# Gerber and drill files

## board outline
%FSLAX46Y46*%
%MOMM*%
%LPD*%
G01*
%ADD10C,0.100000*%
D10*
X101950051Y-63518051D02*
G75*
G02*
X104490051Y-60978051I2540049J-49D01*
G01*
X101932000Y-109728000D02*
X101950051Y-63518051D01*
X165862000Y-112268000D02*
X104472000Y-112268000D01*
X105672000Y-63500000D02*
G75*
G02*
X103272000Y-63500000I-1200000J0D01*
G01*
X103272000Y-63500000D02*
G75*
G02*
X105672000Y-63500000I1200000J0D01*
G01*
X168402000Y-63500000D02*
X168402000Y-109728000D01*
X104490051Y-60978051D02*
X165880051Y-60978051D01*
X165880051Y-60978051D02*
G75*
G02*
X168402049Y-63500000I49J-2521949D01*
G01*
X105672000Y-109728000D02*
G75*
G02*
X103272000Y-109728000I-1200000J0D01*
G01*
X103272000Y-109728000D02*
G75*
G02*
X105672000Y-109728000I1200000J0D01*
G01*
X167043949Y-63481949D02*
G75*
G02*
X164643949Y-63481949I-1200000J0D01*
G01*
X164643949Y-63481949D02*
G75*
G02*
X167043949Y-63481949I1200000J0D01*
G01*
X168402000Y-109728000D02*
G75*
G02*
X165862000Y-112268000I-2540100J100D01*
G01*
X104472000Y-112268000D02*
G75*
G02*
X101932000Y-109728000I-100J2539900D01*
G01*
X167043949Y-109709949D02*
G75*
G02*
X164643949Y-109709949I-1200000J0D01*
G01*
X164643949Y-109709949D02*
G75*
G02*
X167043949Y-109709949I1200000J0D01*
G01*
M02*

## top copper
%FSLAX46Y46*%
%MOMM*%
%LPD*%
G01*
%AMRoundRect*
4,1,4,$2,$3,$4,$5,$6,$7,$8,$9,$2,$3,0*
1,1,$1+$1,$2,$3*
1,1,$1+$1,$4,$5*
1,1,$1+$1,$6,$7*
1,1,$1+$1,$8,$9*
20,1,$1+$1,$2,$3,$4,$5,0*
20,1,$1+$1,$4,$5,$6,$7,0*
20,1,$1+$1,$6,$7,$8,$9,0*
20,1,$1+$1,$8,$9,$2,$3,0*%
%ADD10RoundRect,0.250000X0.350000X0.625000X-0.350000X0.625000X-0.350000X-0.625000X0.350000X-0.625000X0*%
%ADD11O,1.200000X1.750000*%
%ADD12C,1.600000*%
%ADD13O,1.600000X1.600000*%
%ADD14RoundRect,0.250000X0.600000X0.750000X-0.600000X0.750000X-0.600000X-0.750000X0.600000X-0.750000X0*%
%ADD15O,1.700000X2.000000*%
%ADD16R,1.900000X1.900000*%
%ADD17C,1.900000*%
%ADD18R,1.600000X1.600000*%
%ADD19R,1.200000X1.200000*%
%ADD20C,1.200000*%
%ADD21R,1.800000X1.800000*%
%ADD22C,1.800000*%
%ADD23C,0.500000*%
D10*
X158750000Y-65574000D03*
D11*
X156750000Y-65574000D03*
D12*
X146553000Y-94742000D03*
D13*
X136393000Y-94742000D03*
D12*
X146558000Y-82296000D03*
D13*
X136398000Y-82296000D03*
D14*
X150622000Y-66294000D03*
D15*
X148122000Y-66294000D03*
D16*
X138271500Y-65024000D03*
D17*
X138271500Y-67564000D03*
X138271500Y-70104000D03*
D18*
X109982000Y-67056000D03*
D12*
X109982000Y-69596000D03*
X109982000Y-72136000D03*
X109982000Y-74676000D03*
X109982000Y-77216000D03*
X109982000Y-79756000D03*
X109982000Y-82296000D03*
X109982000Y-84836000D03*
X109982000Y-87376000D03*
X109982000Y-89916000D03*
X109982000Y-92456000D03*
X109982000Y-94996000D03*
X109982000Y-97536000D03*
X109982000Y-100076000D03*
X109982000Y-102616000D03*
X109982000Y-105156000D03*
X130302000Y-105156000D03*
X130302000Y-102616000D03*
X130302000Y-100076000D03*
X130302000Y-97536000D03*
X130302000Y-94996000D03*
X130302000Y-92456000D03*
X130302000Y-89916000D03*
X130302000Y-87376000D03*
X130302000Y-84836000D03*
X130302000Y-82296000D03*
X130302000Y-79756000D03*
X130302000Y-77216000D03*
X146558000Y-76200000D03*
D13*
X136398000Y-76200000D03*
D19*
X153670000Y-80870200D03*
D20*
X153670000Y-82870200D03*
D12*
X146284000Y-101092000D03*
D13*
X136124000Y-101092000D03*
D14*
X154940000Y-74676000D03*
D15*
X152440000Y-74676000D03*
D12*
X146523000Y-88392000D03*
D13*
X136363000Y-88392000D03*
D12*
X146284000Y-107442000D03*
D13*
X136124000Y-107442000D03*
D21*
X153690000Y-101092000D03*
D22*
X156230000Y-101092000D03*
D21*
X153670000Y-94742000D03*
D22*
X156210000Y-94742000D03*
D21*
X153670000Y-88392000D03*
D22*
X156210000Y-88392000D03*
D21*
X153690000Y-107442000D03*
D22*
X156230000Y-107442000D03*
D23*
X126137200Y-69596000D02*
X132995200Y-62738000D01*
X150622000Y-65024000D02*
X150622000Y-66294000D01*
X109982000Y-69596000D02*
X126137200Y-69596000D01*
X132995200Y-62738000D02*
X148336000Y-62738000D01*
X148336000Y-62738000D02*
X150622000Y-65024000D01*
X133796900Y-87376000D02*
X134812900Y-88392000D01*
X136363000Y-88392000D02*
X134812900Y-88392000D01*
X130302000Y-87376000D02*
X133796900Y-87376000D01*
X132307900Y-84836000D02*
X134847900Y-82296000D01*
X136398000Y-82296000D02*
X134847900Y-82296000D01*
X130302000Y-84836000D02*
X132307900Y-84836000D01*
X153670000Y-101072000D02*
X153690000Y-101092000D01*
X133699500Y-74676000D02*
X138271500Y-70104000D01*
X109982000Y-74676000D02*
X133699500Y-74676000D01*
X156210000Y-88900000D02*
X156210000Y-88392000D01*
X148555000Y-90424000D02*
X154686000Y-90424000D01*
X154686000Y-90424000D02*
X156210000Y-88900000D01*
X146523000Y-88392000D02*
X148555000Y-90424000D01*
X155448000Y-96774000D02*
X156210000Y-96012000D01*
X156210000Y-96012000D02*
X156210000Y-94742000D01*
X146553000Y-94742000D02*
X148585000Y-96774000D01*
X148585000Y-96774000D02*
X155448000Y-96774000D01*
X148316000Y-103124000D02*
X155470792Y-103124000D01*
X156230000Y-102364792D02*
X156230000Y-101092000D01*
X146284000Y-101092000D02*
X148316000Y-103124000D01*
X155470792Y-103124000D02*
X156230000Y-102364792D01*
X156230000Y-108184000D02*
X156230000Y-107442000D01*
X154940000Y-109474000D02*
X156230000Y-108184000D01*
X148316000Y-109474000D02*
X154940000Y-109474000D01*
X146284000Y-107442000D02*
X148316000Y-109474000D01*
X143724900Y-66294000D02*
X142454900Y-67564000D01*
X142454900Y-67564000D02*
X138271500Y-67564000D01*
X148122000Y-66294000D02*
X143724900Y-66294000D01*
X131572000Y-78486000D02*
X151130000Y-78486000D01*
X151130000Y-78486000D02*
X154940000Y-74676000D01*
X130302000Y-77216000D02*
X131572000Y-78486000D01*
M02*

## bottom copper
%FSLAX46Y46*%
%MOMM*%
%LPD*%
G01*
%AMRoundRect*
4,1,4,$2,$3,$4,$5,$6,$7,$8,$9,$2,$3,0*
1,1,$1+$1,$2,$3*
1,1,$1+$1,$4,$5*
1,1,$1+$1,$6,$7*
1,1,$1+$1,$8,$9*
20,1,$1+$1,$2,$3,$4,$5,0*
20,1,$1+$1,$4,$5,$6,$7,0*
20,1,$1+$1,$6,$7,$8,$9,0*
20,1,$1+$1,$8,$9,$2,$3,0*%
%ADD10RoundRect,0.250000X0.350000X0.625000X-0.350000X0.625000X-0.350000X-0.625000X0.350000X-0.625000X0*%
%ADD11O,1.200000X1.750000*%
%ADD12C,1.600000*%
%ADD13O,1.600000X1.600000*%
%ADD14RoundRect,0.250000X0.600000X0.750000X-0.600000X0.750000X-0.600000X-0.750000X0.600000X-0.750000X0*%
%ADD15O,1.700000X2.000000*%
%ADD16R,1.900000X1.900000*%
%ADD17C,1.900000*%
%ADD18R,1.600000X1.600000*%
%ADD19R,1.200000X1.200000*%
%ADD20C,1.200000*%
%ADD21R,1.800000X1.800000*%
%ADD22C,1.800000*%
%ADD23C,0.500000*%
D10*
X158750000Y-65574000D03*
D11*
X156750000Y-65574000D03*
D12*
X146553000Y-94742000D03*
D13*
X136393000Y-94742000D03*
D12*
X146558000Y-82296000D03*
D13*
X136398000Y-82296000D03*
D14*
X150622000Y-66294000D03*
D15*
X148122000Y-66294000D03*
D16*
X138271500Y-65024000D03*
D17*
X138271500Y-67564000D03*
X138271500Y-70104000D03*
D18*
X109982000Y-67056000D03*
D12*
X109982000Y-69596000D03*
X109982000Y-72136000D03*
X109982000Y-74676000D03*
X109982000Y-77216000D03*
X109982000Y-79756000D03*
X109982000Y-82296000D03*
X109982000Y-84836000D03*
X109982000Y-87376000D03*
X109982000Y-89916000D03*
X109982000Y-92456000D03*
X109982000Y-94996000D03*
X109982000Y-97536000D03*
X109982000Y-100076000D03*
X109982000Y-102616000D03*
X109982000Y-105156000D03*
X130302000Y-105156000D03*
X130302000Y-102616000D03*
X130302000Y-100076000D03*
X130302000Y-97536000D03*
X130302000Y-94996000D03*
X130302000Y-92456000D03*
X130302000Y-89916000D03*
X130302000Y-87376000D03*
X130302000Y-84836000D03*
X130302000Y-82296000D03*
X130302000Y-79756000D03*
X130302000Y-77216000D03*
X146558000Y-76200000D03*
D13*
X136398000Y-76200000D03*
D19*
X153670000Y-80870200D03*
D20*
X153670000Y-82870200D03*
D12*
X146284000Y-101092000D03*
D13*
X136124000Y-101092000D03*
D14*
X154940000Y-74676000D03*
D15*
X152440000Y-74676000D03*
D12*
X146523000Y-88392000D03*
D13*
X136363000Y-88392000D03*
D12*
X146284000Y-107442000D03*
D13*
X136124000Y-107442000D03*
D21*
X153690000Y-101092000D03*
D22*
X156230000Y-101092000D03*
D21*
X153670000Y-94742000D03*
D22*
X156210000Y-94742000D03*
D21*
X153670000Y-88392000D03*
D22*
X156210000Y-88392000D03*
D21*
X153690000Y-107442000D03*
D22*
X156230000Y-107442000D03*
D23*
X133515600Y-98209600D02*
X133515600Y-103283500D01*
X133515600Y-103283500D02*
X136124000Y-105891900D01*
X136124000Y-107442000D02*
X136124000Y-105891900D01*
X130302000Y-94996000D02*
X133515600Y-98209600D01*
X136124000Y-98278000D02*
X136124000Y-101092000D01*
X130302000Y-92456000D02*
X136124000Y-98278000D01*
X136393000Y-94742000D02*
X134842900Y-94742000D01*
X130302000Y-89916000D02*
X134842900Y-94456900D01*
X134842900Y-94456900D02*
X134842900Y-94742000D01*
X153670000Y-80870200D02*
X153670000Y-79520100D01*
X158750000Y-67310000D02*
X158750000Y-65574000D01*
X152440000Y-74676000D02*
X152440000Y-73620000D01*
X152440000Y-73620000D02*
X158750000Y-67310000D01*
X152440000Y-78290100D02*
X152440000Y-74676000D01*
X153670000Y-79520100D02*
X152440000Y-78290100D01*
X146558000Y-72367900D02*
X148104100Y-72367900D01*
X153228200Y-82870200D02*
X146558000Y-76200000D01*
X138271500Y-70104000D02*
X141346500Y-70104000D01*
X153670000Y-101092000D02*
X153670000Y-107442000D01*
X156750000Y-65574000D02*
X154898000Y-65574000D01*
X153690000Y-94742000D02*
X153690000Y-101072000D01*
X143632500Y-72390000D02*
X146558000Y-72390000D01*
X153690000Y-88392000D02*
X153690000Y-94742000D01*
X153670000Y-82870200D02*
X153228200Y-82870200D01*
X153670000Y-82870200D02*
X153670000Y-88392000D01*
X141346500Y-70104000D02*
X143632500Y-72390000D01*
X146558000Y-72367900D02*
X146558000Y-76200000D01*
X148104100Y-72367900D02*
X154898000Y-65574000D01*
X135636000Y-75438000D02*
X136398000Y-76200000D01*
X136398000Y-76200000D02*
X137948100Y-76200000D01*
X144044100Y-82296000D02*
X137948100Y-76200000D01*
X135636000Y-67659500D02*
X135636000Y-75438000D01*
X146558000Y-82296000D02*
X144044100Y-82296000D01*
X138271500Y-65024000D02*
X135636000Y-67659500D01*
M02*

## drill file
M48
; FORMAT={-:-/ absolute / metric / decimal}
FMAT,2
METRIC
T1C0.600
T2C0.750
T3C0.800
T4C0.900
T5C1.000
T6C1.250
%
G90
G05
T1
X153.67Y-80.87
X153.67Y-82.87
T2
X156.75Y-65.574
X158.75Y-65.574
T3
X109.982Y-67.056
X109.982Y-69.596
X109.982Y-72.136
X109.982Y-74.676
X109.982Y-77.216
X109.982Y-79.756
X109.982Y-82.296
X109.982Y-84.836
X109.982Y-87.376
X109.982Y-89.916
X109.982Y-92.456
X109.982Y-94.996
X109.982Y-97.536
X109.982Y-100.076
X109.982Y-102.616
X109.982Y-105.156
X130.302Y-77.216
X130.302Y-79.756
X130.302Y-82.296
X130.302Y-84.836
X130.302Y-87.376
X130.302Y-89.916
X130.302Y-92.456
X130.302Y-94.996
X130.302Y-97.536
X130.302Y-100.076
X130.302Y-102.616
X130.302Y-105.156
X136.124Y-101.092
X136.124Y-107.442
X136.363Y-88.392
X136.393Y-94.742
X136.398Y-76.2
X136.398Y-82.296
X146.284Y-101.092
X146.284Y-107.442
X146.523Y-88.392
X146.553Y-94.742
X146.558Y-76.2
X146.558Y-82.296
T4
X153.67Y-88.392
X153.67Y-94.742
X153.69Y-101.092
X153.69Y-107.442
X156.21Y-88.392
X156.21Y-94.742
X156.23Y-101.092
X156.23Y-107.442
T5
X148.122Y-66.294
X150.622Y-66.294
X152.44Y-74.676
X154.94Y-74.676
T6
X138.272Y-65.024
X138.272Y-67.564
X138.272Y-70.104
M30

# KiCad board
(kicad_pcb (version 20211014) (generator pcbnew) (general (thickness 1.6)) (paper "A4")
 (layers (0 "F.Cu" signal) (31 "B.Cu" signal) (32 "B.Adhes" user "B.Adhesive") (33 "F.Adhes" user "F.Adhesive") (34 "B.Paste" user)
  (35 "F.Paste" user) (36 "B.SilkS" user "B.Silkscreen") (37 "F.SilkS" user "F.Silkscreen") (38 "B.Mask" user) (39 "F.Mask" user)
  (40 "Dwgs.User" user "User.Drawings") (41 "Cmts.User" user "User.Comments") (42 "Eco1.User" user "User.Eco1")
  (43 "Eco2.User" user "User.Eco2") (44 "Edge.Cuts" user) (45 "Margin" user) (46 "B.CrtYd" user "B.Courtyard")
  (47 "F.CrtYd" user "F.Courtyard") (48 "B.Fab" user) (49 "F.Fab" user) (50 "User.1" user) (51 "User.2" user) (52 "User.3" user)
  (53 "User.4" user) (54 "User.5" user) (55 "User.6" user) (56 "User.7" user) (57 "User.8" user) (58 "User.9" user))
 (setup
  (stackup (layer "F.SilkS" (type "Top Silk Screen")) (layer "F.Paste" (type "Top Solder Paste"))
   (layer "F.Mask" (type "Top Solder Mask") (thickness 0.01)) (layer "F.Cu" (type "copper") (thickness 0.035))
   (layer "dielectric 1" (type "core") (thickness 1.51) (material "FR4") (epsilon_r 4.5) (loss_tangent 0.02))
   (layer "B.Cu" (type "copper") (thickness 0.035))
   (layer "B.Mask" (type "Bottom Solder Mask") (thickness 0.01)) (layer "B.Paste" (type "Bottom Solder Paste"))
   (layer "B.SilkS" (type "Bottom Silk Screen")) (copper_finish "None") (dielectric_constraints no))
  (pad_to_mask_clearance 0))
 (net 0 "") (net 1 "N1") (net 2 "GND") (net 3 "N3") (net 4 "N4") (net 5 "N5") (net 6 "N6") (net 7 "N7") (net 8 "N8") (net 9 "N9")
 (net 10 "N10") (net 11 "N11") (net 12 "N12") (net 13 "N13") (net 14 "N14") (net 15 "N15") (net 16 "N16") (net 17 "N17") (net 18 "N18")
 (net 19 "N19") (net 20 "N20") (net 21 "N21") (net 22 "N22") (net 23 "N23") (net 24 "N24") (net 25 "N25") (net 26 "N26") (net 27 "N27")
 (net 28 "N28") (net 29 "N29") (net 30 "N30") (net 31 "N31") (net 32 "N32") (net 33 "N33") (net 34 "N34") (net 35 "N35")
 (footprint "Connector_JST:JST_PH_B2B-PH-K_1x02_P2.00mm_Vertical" (layer "F.Cu") (at 158.75 65.574 180)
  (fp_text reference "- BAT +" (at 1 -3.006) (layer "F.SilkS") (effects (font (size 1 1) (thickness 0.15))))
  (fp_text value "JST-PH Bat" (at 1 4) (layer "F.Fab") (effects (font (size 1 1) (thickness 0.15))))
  (pad "1" thru_hole roundrect (at 0 0 180) (size 1.2 1.75) (drill 0.75) (layers *.Cu *.Mask) (roundrect_rratio 0.208333) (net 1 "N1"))
  (pad "2" thru_hole oval (at 2 0 180) (size 1.2 1.75) (drill 0.75) (layers *.Cu *.Mask) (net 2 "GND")))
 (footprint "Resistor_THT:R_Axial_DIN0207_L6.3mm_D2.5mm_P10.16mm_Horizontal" (layer "F.Cu") (at 146.553 94.742 180)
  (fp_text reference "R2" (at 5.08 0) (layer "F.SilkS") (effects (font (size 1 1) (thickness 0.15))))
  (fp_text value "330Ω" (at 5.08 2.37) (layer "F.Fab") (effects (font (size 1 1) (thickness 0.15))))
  (pad "1" thru_hole circle (at 0 0 180) (size 1.6 1.6) (drill 0.8) (layers *.Cu *.Mask) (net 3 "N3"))
  (pad "2" thru_hole oval (at 10.16 0 180) (size 1.6 1.6) (drill 0.8) (layers *.Cu *.Mask) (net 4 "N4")))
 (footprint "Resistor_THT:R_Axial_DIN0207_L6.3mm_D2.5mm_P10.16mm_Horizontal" (layer "F.Cu") (at 146.558 82.296 180)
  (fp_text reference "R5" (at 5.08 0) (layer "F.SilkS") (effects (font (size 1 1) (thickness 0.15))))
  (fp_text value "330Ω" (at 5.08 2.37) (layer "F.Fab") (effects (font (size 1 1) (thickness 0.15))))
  (pad "1" thru_hole circle (at 0 0 180) (size 1.6 1.6) (drill 0.8) (layers *.Cu *.Mask) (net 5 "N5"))
  (pad "2" thru_hole oval (at 10.16 0 180) (size 1.6 1.6) (drill 0.8) (layers *.Cu *.Mask) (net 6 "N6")))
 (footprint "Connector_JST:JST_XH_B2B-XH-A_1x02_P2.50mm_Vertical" (layer "F.Cu") (at 150.622 66.294 180)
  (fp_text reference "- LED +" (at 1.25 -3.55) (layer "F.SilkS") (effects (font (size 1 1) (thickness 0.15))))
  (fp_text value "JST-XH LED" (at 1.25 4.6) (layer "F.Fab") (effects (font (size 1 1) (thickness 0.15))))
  (pad "1" thru_hole roundrect (at 0 0 180) (size 1.7 2) (drill 1) (layers *.Cu *.Mask) (roundrect_rratio 0.147059) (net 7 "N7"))
  (pad "2" thru_hole oval (at 2.5 0 180) (size 1.7 2) (drill 1) (layers *.Cu *.Mask) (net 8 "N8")))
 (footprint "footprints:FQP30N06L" (layer "F.Cu") (at 138.684 67.564)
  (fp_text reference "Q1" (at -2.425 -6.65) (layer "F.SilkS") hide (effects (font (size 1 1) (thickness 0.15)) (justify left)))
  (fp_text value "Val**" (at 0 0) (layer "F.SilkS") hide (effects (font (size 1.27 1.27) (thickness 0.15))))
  (pad "1" thru_hole rect (at -0.4125 -2.54) (size 1.9 1.9) (drill 1.25) (layers *.Cu *.Mask) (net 5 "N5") (thermal_width 0.45))
  (pad "2" thru_hole circle (at -0.4125 0) (size 1.9 1.9) (drill 1.25) (layers *.Cu *.Mask) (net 8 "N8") (thermal_width 0.45))
  (pad "3" thru_hole circle (at -0.4125 2.54) (size 1.9 1.9) (drill 1.25) (layers *.Cu *.Mask) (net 2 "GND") (thermal_width 0.45)))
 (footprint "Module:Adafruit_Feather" (layer "F.Cu") (at 109.982 67.056)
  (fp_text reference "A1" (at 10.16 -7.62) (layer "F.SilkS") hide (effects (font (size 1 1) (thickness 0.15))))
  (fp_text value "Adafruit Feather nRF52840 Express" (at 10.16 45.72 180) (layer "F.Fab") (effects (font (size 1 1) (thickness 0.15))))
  (pad "1" thru_hole rect (at 0 0 180) (size 1.6 1.6) (drill 0.8) (layers *.Cu *.Mask) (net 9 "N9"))
  (pad "2" thru_hole circle (at 0 2.54 180) (size 1.6 1.6) (drill 0.8) (layers *.Cu *.Mask) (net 7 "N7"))
  (pad "3" thru_hole circle (at 0 5.08 180) (size 1.6 1.6) (drill 0.8) (layers *.Cu *.Mask) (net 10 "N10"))
  (pad "4" thru_hole circle (at 0 7.62 180) (size 1.6 1.6) (drill 0.8) (layers *.Cu *.Mask) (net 2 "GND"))
  (pad "5" thru_hole circle (at 0 10.16 180) (size 1.6 1.6) (drill 0.8) (layers *.Cu *.Mask) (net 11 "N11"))
  (pad "6" thru_hole circle (at 0 12.7 180) (size 1.6 1.6) (drill 0.8) (layers *.Cu *.Mask) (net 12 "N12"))
  (pad "7" thru_hole circle (at 0 15.24 180) (size 1.6 1.6) (drill 0.8) (layers *.Cu *.Mask) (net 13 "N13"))
  (pad "8" thru_hole circle (at 0 17.78 180) (size 1.6 1.6) (drill 0.8) (layers *.Cu *.Mask) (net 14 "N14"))
  (pad "9" thru_hole circle (at 0 20.32 180) (size 1.6 1.6) (drill 0.8) (layers *.Cu *.Mask) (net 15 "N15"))
  (pad "10" thru_hole circle (at 0 22.86 180) (size 1.6 1.6) (drill 0.8) (layers *.Cu *.Mask) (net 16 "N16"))
  (pad "11" thru_hole circle (at 0 25.4 180) (size 1.6 1.6) (drill 0.8) (layers *.Cu *.Mask) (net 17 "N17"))
  (pad "12" thru_hole circle (at 0 27.94 180) (size 1.6 1.6) (drill 0.8) (layers *.Cu *.Mask) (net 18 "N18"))
  (pad "13" thru_hole circle (at 0 30.48 180) (size 1.6 1.6) (drill 0.8) (layers *.Cu *.Mask) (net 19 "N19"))
  (pad "14" thru_hole circle (at 0 33.02 180) (size 1.6 1.6) (drill 0.8) (layers *.Cu *.Mask) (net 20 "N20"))
  (pad "15" thru_hole circle (at 0 35.56 180) (size 1.6 1.6) (drill 0.8) (layers *.Cu *.Mask) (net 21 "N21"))
  (pad "16" thru_hole circle (at 0 38.1 180) (size 1.6 1.6) (drill 0.8) (layers *.Cu *.Mask) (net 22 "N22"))
  (pad "17" thru_hole circle (at 20.32 38.1 180) (size 1.6 1.6) (drill 0.8) (layers *.Cu *.Mask) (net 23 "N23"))
  (pad "18" thru_hole circle (at 20.32 35.56 180) (size 1.6 1.6) (drill 0.8) (layers *.Cu *.Mask) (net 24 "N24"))
  (pad "19" thru_hole circle (at 20.32 33.02 180) (size 1.6 1.6) (drill 0.8) (layers *.Cu *.Mask) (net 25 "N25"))
  (pad "20" thru_hole circle (at 20.32 30.48 180) (size 1.6 1.6) (drill 0.8) (layers *.Cu *.Mask) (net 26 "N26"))
  (pad "21" thru_hole circle (at 20.32 27.94 180) (size 1.6 1.6) (drill 0.8) (layers *.Cu *.Mask) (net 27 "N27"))
  (pad "22" thru_hole circle (at 20.32 25.4 180) (size 1.6 1.6) (drill 0.8) (layers *.Cu *.Mask) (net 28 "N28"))
  (pad "23" thru_hole circle (at 20.32 22.86 180) (size 1.6 1.6) (drill 0.8) (layers *.Cu *.Mask) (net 4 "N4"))
  (pad "24" thru_hole circle (at 20.32 20.32 180) (size 1.6 1.6) (drill 0.8) (layers *.Cu *.Mask) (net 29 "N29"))
  (pad "25" thru_hole circle (at 20.32 17.78 180) (size 1.6 1.6) (drill 0.8) (layers *.Cu *.Mask) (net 6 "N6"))
  (pad "26" thru_hole circle (at 20.32 15.24 180) (size 1.6 1.6) (drill 0.8) (layers *.Cu *.Mask) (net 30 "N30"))
  (pad "27" thru_hole circle (at 20.32 12.7 180) (size 1.6 1.6) (drill 0.8) (layers *.Cu *.Mask) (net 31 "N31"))
  (pad "28" thru_hole circle (at 20.32 10.16 180) (size 1.6 1.6) (drill 0.8) (layers *.Cu *.Mask) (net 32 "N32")))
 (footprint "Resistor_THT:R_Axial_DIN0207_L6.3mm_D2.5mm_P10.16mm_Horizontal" (layer "F.Cu") (at 146.558 76.2 180)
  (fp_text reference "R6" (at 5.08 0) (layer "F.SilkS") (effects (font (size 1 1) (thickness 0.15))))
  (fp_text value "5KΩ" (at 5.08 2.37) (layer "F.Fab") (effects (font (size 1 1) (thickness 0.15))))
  (pad "1" thru_hole circle (at 0 0 180) (size 1.6 1.6) (drill 0.8) (layers *.Cu *.Mask) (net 2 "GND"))
  (pad "2" thru_hole oval (at 10.16 0 180) (size 1.6 1.6) (drill 0.8) (layers *.Cu *.Mask) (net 5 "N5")))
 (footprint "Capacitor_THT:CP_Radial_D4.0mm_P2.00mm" (layer "F.Cu") (at 153.67 80.8702 -90)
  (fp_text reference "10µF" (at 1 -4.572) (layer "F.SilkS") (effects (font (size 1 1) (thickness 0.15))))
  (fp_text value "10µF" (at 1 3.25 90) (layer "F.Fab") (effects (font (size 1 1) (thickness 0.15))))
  (pad "1" thru_hole rect (at 0 0 270) (size 1.2 1.2) (drill 0.6) (layers *.Cu *.Mask) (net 1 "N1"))
  (pad "2" thru_hole circle (at 2 0 270) (size 1.2 1.2) (drill 0.6) (layers *.Cu *.Mask) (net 2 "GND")))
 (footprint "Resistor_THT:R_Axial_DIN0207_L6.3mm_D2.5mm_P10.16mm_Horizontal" (layer "F.Cu") (at 146.284 101.092 180)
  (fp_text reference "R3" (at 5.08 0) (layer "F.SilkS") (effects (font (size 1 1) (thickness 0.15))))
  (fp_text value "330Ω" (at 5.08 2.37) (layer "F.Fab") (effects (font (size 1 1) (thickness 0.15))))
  (pad "1" thru_hole circle (at 0 0 180) (size 1.6 1.6) (drill 0.8) (layers *.Cu *.Mask) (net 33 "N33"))
  (pad "2" thru_hole oval (at 10.16 0 180) (size 1.6 1.6) (drill 0.8) (layers *.Cu *.Mask) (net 28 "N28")))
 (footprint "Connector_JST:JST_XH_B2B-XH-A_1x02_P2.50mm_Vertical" (layer "F.Cu") (at 154.94 74.676 180)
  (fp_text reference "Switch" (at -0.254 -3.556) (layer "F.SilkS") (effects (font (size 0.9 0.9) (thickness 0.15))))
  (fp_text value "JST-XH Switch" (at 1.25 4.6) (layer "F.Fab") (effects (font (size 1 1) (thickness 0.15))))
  (pad "1" thru_hole roundrect (at 0 0 180) (size 1.7 2) (drill 1) (layers *.Cu *.Mask) (roundrect_rratio 0.147059) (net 32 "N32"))
  (pad "2" thru_hole oval (at 2.5 0 180) (size 1.7 2) (drill 1) (layers *.Cu *.Mask) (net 1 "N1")))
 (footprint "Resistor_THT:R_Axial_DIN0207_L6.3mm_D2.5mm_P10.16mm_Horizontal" (layer "F.Cu") (at 146.523 88.392 180)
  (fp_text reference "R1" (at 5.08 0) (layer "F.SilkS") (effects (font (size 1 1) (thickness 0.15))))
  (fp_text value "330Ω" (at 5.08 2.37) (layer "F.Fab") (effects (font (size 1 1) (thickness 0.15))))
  (pad "1" thru_hole circle (at 0 0 180) (size 1.6 1.6) (drill 0.8) (layers *.Cu *.Mask) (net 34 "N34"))
  (pad "2" thru_hole oval (at 10.16 0 180) (size 1.6 1.6) (drill 0.8) (layers *.Cu *.Mask) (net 29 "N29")))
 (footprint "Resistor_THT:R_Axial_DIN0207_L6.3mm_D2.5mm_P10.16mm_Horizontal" (layer "F.Cu") (at 146.284 107.442 180)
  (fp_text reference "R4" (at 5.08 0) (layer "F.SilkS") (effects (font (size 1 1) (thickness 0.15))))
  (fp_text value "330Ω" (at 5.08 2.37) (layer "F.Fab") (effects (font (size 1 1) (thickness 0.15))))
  (pad "1" thru_hole circle (at 0 0 180) (size 1.6 1.6) (drill 0.8) (layers *.Cu *.Mask) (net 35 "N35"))
  (pad "2" thru_hole oval (at 10.16 0 180) (size 1.6 1.6) (drill 0.8) (layers *.Cu *.Mask) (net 27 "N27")))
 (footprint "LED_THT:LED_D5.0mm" (layer "B.Cu") (at 153.69 101.092)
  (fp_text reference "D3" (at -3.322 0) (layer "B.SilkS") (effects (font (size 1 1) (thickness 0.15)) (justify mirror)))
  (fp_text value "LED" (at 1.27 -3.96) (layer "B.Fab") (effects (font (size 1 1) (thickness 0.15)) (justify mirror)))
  (pad "1" thru_hole rect (at 0 0) (size 1.8 1.8) (drill 0.9) (layers *.Cu *.Mask) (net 2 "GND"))
  (pad "2" thru_hole circle (at 2.54 0) (size 1.8 1.8) (drill 0.9) (layers *.Cu *.Mask) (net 33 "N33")))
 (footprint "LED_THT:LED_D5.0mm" (layer "B.Cu") (at 153.67 94.742)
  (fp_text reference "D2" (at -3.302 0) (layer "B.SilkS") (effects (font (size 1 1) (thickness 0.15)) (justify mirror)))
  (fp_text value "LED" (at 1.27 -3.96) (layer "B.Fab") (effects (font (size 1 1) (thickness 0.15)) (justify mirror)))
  (pad "1" thru_hole rect (at 0 0) (size 1.8 1.8) (drill 0.9) (layers *.Cu *.Mask) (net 2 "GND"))
  (pad "2" thru_hole circle (at 2.54 0) (size 1.8 1.8) (drill 0.9) (layers *.Cu *.Mask) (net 3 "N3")))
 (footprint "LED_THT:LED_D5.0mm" (layer "B.Cu") (at 153.67 88.392)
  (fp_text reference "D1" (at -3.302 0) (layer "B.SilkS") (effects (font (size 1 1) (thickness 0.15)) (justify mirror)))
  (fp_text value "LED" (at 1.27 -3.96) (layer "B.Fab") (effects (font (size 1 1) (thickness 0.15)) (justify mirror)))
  (pad "1" thru_hole rect (at 0 0) (size 1.8 1.8) (drill 0.9) (layers *.Cu *.Mask) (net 2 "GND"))
  (pad "2" thru_hole circle (at 2.54 0) (size 1.8 1.8) (drill 0.9) (layers *.Cu *.Mask) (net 34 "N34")))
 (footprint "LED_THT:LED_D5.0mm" (layer "B.Cu") (at 153.69 107.442)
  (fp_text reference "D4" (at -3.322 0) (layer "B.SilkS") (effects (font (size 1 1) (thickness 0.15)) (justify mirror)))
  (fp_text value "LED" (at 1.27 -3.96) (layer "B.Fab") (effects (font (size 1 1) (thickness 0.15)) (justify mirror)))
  (pad "1" thru_hole rect (at 0 0) (size 1.8 1.8) (drill 0.9) (layers *.Cu *.Mask) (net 2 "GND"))
  (pad "2" thru_hole circle (at 2.54 0) (size 1.8 1.8) (drill 0.9) (layers *.Cu *.Mask) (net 35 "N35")))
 (gr_arc (start 101.950051 63.518051) (mid 102.694 61.722) (end 104.490051 60.978051) (layer "Edge.Cuts") (width 0.1))
 (gr_line (start 101.932 109.728) (end 101.950051 63.518051) (layer "Edge.Cuts") (width 0.1))
 (gr_line (start 165.862 112.268) (end 104.472 112.268) (layer "Edge.Cuts") (width 0.1))
 (gr_circle (center 104.472 63.5) (end 105.672 63.5) (layer "Edge.Cuts") (width 0.1) (fill none))
 (gr_line (start 168.402 63.5) (end 168.402 109.728) (layer "Edge.Cuts") (width 0.1))
 (gr_line (start 104.490051 60.978051) (end 165.880051 60.978051) (layer "Edge.Cuts") (width 0.1))
 (gr_arc (start 165.880051 60.978051) (mid 167.663352 61.716699) (end 168.402 63.5) (layer "Edge.Cuts") (width 0.1))
 (gr_circle (center 104.472 109.728) (end 105.672 109.728) (layer "Edge.Cuts") (width 0.1) (fill none))
 (gr_circle (center 165.843949 63.481949) (end 167.043949 63.481949) (layer "Edge.Cuts") (width 0.1) (fill none))
 (gr_arc (start 168.402 109.728) (mid 167.658034 111.52402) (end 165.862 112.268) (layer "Edge.Cuts") (width 0.1))
 (gr_arc (start 104.472 112.268) (mid 102.6759 111.524072) (end 101.932 109.728) (layer "Edge.Cuts") (width 0.1))
 (gr_circle (center 165.843949 109.709949) (end 167.043949 109.709949) (layer "Edge.Cuts") (width 0.1) (fill none))
 (segment (start 126.1372 69.596) (end 132.9952 62.738) (width 0.5) (layer "F.Cu") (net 7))
 (segment (start 150.622 65.024) (end 150.622 66.294) (width 0.5) (layer "F.Cu") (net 7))
 (segment (start 109.982 69.596) (end 126.1372 69.596) (width 0.5) (layer "F.Cu") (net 7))
 (segment (start 132.9952 62.738) (end 148.336 62.738) (width 0.5) (layer "F.Cu") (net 7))
 (segment (start 148.336 62.738) (end 150.622 65.024) (width 0.5) (layer "F.Cu") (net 7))
 (segment (start 133.5156 98.2096) (end 133.5156 103.2835) (width 0.5) (layer "B.Cu") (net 27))
 (segment (start 133.5156 103.2835) (end 136.124 105.8919) (width 0.5) (layer "B.Cu") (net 27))
 (segment (start 136.124 107.442) (end 136.124 105.8919) (width 0.5) (layer "B.Cu") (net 27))
 (segment (start 130.302 94.996) (end 133.5156 98.2096) (width 0.5) (layer "B.Cu") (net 27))
 (segment (start 136.124 98.278) (end 136.124 101.092) (width 0.5) (layer "B.Cu") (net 28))
 (segment (start 130.302 92.456) (end 136.124 98.278) (width 0.5) (layer "B.Cu") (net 28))
 (segment (start 136.393 94.742) (end 134.8429 94.742) (width 0.5) (layer "B.Cu") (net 4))
 (segment (start 130.302 89.916) (end 134.8429 94.4569) (width 0.5) (layer "B.Cu") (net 4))
 (segment (start 134.8429 94.4569) (end 134.8429 94.742) (width 0.5) (layer "B.Cu") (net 4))
 (segment (start 133.7969 87.376) (end 134.8129 88.392) (width 0.5) (layer "F.Cu") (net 29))
 (segment (start 136.363 88.392) (end 134.8129 88.392) (width 0.5) (layer "F.Cu") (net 29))
 (segment (start 130.302 87.376) (end 133.7969 87.376) (width 0.5) (layer "F.Cu") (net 29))
 (segment (start 132.3079 84.836) (end 134.8479 82.296) (width 0.5) (layer "F.Cu") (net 6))
 (segment (start 136.398 82.296) (end 134.8479 82.296) (width 0.5) (layer "F.Cu") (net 6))
 (segment (start 130.302 84.836) (end 132.3079 84.836) (width 0.5) (layer "F.Cu") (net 6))
 (segment (start 153.67 80.8702) (end 153.67 79.5201) (width 0.5) (layer "B.Cu") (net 1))
 (segment (start 158.75 67.31) (end 158.75 65.574) (width 0.5) (layer "B.Cu") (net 1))
 (segment (start 152.44 74.676) (end 152.44 73.62) (width 0.5) (layer "B.Cu") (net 1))
 (segment (start 152.44 73.62) (end 158.75 67.31) (width 0.5) (layer "B.Cu") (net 1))
 (segment (start 152.44 78.2901) (end 152.44 74.676) (width 0.5) (layer "B.Cu") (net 1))
 (segment (start 153.67 79.5201) (end 152.44 78.2901) (width 0.5) (layer "B.Cu") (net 1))
 (segment (start 153.67 101.072) (end 153.69 101.092) (width 0.5) (layer "F.Cu") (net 2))
 (segment (start 133.6995 74.676) (end 138.2715 70.104) (width 0.5) (layer "F.Cu") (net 2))
 (segment (start 109.982 74.676) (end 133.6995 74.676) (width 0.5) (layer "F.Cu") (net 2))
 (segment (start 146.558 72.3679) (end 148.1041 72.3679) (width 0.5) (layer "B.Cu") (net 2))
 (segment (start 153.2282 82.8702) (end 146.558 76.2) (width 0.5) (layer "B.Cu") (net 2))
 (segment (start 138.2715 70.104) (end 141.3465 70.104) (width 0.5) (layer "B.Cu") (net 2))
 (segment (start 153.67 101.092) (end 153.67 107.442) (width 0.5) (layer "B.Cu") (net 2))
 (segment (start 156.75 65.574) (end 154.898 65.574) (width 0.5) (layer "B.Cu") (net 2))
 (segment (start 153.69 94.742) (end 153.69 101.072) (width 0.5) (layer "B.Cu") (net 2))
 (segment (start 143.6325 72.39) (end 146.558 72.39) (width 0.5) (layer "B.Cu") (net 2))
 (segment (start 153.69 88.392) (end 153.69 94.742) (width 0.5) (layer "B.Cu") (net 2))
 (segment (start 153.67 82.8702) (end 153.2282 82.8702) (width 0.5) (layer "B.Cu") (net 2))
 (segment (start 153.67 82.8702) (end 153.67 88.392) (width 0.5) (layer "B.Cu") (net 2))
 (segment (start 141.3465 70.104) (end 143.6325 72.39) (width 0.5) (layer "B.Cu") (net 2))
 (segment (start 146.558 72.3679) (end 146.558 76.2) (width 0.5) (layer "B.Cu") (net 2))
 (segment (start 148.1041 72.3679) (end 154.898 65.574) (width 0.5) (layer "B.Cu") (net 2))
 (segment (start 156.21 88.9) (end 156.21 88.392) (width 0.5) (layer "F.Cu") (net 34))
 (segment (start 148.555 90.424) (end 154.686 90.424) (width 0.5) (layer "F.Cu") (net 34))
 (segment (start 154.686 90.424) (end 156.21 88.9) (width 0.5) (layer "F.Cu") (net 34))
 (segment (start 146.523 88.392) (end 148.555 90.424) (width 0.5) (layer "F.Cu") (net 34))
 (segment (start 155.448 96.774) (end 156.21 96.012) (width 0.5) (layer "F.Cu") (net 3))
 (segment (start 156.21 96.012) (end 156.21 94.742) (width 0.5) (layer "F.Cu") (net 3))
 (segment (start 146.553 94.742) (end 148.585 96.774) (width 0.5) (layer "F.Cu") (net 3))
 (segment (start 148.585 96.774) (end 155.448 96.774) (width 0.5) (layer "F.Cu") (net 3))
 (segment (start 148.316 103.124) (end 155.470792 103.124) (width 0.5) (layer "F.Cu") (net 33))
 (segment (start 156.23 102.364792) (end 156.23 101.092) (width 0.5) (layer "F.Cu") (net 33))
 (segment (start 146.284 101.092) (end 148.316 103.124) (width 0.5) (layer "F.Cu") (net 33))
 (segment (start 155.470792 103.124) (end 156.23 102.364792) (width 0.5) (layer "F.Cu") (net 33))
 (segment (start 156.23 108.184) (end 156.23 107.442) (width 0.5) (layer "F.Cu") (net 35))
 (segment (start 154.94 109.474) (end 156.23 108.184) (width 0.5) (layer "F.Cu") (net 35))
 (segment (start 148.316 109.474) (end 154.94 109.474) (width 0.5) (layer "F.Cu") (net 35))
 (segment (start 146.284 107.442) (end 148.316 109.474) (width 0.5) (layer "F.Cu") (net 35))
 (segment (start 143.7249 66.294) (end 142.4549 67.564) (width 0.5) (layer "F.Cu") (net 8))
 (segment (start 142.4549 67.564) (end 138.2715 67.564) (width 0.5) (layer "F.Cu") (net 8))
 (segment (start 148.122 66.294) (end 143.7249 66.294) (width 0.5) (layer "F.Cu") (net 8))
 (segment (start 135.636 75.438) (end 136.398 76.2) (width 0.5) (layer "B.Cu") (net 5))
 (segment (start 136.398 76.2) (end 137.9481 76.2) (width 0.5) (layer "B.Cu") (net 5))
 (segment (start 144.0441 82.296) (end 137.9481 76.2) (width 0.5) (layer "B.Cu") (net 5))
 (segment (start 135.636 67.6595) (end 135.636 75.438) (width 0.5) (layer "B.Cu") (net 5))
 (segment (start 146.558 82.296) (end 144.0441 82.296) (width 0.5) (layer "B.Cu") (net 5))
 (segment (start 138.2715 65.024) (end 135.636 67.6595) (width 0.5) (layer "B.Cu") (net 5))
 (segment (start 131.572 78.486) (end 151.13 78.486) (width 0.5) (layer "F.Cu") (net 32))
 (segment (start 151.13 78.486) (end 154.94 74.676) (width 0.5) (layer "F.Cu") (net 32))
 (segment (start 130.302 77.216) (end 131.572 78.486) (width 0.5) (layer "F.Cu") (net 32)))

